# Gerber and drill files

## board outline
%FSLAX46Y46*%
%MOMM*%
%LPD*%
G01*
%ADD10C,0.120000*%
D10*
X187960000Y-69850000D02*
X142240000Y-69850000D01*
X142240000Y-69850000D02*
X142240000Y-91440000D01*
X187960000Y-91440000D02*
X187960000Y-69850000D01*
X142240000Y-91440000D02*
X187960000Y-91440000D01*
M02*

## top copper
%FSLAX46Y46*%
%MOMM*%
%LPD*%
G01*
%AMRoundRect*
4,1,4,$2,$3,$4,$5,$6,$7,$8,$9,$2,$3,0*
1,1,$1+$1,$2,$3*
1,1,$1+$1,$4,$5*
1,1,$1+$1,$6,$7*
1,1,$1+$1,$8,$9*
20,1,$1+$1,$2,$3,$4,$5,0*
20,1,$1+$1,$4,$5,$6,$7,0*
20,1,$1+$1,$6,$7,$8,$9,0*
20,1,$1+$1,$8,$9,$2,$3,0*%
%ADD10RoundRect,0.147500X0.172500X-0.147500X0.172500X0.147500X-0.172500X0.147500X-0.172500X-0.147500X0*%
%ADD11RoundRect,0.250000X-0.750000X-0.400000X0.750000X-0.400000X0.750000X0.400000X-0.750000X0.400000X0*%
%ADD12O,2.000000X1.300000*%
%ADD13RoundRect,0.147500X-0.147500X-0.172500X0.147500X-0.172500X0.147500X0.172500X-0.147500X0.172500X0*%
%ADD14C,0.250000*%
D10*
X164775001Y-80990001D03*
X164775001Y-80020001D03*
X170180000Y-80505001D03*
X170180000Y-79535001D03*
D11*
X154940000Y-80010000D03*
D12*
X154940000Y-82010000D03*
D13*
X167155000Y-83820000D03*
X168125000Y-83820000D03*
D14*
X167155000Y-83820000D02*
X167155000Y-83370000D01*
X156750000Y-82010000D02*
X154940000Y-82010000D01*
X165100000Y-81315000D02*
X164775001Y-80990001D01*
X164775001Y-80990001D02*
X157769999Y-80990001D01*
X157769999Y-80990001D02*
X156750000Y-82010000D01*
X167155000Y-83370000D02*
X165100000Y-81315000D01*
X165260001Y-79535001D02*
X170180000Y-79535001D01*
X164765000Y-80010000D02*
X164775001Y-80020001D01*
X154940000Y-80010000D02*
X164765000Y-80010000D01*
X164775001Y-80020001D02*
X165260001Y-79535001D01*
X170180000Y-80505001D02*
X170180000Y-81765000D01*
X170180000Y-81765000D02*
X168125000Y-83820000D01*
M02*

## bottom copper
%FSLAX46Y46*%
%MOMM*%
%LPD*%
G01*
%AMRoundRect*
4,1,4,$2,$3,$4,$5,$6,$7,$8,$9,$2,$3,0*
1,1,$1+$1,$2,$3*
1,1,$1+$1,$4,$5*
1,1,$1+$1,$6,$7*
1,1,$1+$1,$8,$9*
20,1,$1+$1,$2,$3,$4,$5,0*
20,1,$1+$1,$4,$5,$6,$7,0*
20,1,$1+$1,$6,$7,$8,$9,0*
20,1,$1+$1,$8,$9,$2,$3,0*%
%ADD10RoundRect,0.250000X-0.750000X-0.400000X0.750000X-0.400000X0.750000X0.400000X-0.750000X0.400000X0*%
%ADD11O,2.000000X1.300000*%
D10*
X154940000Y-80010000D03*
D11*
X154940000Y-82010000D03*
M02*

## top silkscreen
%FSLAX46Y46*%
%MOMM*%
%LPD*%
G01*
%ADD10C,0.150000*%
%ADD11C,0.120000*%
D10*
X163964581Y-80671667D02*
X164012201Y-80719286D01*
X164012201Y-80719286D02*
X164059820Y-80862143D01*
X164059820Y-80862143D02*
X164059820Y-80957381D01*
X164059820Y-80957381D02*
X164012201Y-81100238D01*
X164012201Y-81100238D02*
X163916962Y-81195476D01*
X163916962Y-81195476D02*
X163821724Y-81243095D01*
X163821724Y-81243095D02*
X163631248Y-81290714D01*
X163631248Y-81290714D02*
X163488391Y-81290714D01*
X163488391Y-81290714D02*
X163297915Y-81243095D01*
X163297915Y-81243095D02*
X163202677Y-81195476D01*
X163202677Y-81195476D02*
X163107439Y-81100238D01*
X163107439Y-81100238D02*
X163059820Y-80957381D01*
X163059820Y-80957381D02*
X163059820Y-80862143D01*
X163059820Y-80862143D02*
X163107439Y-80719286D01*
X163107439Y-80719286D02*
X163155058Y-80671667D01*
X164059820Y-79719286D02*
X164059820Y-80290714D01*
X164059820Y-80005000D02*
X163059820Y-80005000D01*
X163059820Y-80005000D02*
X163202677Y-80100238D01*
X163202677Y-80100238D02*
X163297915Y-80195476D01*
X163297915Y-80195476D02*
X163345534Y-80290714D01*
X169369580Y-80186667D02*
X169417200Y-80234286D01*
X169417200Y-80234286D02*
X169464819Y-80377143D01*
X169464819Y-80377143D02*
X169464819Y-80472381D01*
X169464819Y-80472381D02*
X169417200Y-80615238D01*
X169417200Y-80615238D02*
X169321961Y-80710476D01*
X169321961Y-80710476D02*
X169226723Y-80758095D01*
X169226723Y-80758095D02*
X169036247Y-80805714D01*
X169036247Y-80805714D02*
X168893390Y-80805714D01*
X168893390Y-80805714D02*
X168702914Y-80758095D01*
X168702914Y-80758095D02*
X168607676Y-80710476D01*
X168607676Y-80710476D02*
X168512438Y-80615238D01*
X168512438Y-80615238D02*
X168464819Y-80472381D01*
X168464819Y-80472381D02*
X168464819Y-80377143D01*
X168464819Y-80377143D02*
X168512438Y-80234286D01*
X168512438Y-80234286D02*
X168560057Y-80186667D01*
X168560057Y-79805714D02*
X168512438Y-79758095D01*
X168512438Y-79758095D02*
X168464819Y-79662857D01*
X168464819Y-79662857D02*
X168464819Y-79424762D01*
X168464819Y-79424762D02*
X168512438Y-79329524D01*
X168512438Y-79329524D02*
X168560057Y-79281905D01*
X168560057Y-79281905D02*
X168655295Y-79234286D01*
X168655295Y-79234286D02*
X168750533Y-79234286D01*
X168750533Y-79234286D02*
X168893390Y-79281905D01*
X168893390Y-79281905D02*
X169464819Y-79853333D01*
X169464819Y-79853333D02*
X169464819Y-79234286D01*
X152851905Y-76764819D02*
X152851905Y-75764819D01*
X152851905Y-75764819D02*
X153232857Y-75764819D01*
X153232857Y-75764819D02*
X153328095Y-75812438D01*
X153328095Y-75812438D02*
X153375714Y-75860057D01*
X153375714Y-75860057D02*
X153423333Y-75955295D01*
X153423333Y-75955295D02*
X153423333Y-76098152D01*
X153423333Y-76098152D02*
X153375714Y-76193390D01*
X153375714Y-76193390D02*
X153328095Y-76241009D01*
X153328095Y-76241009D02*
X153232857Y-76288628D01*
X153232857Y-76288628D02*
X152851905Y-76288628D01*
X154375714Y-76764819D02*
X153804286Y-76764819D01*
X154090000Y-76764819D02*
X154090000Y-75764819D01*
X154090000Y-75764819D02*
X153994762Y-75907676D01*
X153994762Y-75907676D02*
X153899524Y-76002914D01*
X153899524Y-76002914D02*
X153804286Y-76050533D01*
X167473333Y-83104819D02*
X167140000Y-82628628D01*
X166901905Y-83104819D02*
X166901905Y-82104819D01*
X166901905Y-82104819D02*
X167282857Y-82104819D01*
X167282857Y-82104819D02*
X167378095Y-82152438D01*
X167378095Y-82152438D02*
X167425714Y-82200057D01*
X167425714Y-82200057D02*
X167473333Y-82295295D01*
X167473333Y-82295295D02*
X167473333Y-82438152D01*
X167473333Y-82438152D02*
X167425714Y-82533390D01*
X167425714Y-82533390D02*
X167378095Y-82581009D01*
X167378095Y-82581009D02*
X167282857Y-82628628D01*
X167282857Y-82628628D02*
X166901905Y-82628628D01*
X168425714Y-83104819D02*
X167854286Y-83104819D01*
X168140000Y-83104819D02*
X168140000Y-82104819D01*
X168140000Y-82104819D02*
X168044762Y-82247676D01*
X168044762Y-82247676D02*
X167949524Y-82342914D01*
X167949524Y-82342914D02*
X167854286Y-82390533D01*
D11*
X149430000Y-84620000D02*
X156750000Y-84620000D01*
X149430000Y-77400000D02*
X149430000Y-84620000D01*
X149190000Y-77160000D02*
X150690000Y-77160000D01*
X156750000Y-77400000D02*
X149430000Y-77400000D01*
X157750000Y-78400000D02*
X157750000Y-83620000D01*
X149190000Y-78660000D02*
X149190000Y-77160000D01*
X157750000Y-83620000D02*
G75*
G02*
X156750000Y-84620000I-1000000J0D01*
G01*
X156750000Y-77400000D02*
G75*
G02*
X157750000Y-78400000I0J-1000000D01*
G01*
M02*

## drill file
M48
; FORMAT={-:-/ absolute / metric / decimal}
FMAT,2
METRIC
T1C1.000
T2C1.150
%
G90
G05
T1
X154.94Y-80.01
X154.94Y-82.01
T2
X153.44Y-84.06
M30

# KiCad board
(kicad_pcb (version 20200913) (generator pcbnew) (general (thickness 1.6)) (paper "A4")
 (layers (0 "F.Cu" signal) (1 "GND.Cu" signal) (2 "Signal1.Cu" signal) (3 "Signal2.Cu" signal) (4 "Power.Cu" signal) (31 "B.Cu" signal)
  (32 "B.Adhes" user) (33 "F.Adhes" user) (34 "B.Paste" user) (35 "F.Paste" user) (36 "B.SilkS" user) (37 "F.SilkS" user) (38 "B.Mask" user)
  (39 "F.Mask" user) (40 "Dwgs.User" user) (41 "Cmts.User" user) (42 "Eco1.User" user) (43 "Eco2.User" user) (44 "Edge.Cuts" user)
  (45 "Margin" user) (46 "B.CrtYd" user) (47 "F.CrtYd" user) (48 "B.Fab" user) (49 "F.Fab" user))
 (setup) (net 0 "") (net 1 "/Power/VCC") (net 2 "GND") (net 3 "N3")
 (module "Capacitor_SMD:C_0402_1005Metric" (layer "F.Cu") (at 164.775001 80.505001 90)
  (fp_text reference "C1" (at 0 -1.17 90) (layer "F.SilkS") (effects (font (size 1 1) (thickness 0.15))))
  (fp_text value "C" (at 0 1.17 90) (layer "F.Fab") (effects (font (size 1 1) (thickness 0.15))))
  (pad "1" smd roundrect (at -0.485 0 90) (size 0.59 0.64) (layers "F.Cu" "F.Paste" "F.Mask") (roundrect_rratio 0.25) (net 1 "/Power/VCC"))
  (pad "2" smd roundrect (at 0.485 0 90) (size 0.59 0.64) (layers "F.Cu" "F.Paste" "F.Mask") (roundrect_rratio 0.25) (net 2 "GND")))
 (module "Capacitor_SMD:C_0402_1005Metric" (layer "F.Cu") (at 170.18 80.020001 90)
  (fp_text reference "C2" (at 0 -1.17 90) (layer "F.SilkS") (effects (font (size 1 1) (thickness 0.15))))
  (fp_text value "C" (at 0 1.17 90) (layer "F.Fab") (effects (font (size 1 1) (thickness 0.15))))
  (pad "1" smd roundrect (at -0.485 0 90) (size 0.59 0.64) (layers "F.Cu" "F.Paste" "F.Mask") (roundrect_rratio 0.25) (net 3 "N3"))
  (pad "2" smd roundrect (at 0.485 0 90) (size 0.59 0.64) (layers "F.Cu" "F.Paste" "F.Mask") (roundrect_rratio 0.25) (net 2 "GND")))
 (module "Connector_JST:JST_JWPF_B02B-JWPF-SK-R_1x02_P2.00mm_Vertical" (layer "F.Cu") (at 154.94 80.01)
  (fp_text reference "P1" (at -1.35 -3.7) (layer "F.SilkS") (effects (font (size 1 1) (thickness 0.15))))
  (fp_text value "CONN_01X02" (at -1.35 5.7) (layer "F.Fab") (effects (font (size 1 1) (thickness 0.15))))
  (fp_line (start -5.51 4.61) (end 1.81 4.61) (layer "F.SilkS") (width 0.12))
  (fp_line (start -5.51 -2.61) (end -5.51 4.61) (layer "F.SilkS") (width 0.12))
  (fp_line (start -5.75 -2.85) (end -4.25 -2.85) (layer "F.SilkS") (width 0.12))
  (fp_line (start 1.81 -2.61) (end -5.51 -2.61) (layer "F.SilkS") (width 0.12))
  (fp_line (start 2.81 -1.61) (end 2.81 3.61) (layer "F.SilkS") (width 0.12))
  (fp_line (start -5.75 -1.35) (end -5.75 -2.85) (layer "F.SilkS") (width 0.12))
  (fp_arc (start 1.81 3.61) (end 2.81 3.61) (angle 90) (layer "F.SilkS") (width 0.12))
  (fp_arc (start 1.81 -1.61) (end 1.81 -2.61) (angle 90) (layer "F.SilkS") (width 0.12))
  (pad "" np_thru_hole circle (at -1.5 4.05) (size 1.15 1.15) (drill 1.15) (layers *.Cu *.Mask))
  (pad "1" thru_hole roundrect (at 0 0) (size 2 1.3) (drill 1) (layers *.Cu *.Mask) (roundrect_rratio 0.192308) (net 2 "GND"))
  (pad "2" thru_hole oval (at 0 2) (size 2 1.3) (drill 1) (layers *.Cu *.Mask) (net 1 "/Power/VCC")))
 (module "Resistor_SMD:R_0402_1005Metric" (layer "F.Cu") (at 167.64 83.82)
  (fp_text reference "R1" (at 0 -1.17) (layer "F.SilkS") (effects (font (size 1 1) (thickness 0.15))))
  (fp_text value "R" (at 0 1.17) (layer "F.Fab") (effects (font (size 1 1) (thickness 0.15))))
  (pad "1" smd roundrect (at -0.485 0) (size 0.59 0.64) (layers "F.Cu" "F.Paste" "F.Mask") (roundrect_rratio 0.25) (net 1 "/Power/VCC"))
  (pad "2" smd roundrect (at 0.485 0) (size 0.59 0.64) (layers "F.Cu" "F.Paste" "F.Mask") (roundrect_rratio 0.25) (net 3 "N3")))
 (gr_line (start 187.96 69.85) (end 142.24 69.85) (layer "Edge.Cuts") (width 0.12))
 (gr_line (start 142.24 69.85) (end 142.24 91.44) (layer "Edge.Cuts") (width 0.12))
 (gr_line (start 187.96 91.44) (end 187.96 69.85) (layer "Edge.Cuts") (width 0.12))
 (gr_line (start 142.24 91.44) (end 187.96 91.44) (layer "Edge.Cuts") (width 0.12))
 (segment (start 167.155 83.82) (end 167.155 83.37) (width 0.25) (layer "F.Cu") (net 1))
 (segment (start 156.75 82.01) (end 154.94 82.01) (width 0.25) (layer "F.Cu") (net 1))
 (segment (start 165.1 81.315) (end 164.775001 80.990001) (width 0.25) (layer "F.Cu") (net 1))
 (segment (start 164.775001 80.990001) (end 157.769999 80.990001) (width 0.25) (layer "F.Cu") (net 1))
 (segment (start 157.769999 80.990001) (end 156.75 82.01) (width 0.25) (layer "F.Cu") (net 1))
 (segment (start 167.155 83.37) (end 165.1 81.315) (width 0.25) (layer "F.Cu") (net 1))
 (segment (start 180 88) (end 160 88) (width 0.25) (layer "Signal1.Cu") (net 1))
 (segment (start 179.9848 73) (end 160 73) (width 0.25) (layer "Signal1.Cu") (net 1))
 (segment (start 180 73.0152) (end 179.9848 73) (width 0.25) (layer "Signal1.Cu") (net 1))
 (segment (start 160 88) (end 160 82.0874) (width 0.25) (layer "Signal1.Cu") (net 1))
 (segment (start 180 88) (end 180 73.0152) (width 0.25) (layer "Signal1.Cu") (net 1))
 (segment (start 160 82.0874) (end 160 73) (width 0.25) (layer "Signal1.Cu") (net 1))
 (segment (start 159.9226 82.01) (end 160 82.0874) (width 0.25) (layer "Signal1.Cu") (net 1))
 (segment (start 154.94 82.01) (end 159.9226 82.01) (width 0.25) (layer "Signal1.Cu") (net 1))
 (segment (start 161 82.0314) (end 161 87) (width 0.25) (layer "Power.Cu") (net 1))
 (segment (start 154.94 82.01) (end 160.9786 82.01) (width 0.25) (layer "Power.Cu") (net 1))
 (segment (start 179 86.9888) (end 179 74) (width 0.25) (layer "Power.Cu") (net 1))
 (segment (start 161 74) (end 179 74) (width 0.25) (layer "Power.Cu") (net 1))
 (segment (start 161 87) (end 178.9888 87) (width 0.25) (layer "Power.Cu") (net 1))
 (segment (start 178.9888 87) (end 179 86.9888) (width 0.25) (layer "Power.Cu") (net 1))
 (segment (start 160.9786 82.01) (end 161 82.0314) (width 0.25) (layer "Power.Cu") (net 1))
 (segment (start 161 74) (end 161 82.0314) (width 0.25) (layer "Power.Cu") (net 1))
 (segment (start 165.260001 79.535001) (end 170.18 79.535001) (width 0.25) (layer "F.Cu") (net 2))
 (segment (start 164.765 80.01) (end 164.775001 80.020001) (width 0.25) (layer "F.Cu") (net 2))
 (segment (start 154.94 80.01) (end 164.765 80.01) (width 0.25) (layer "F.Cu") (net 2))
 (segment (start 164.775001 80.020001) (end 165.260001 79.535001) (width 0.25) (layer "F.Cu") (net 2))
 (segment (start 180 73) (end 180 88) (width 0.25) (layer "GND.Cu") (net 2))
 (segment (start 160 73) (end 180 73) (width 0.25) (layer "GND.Cu") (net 2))
 (segment (start 180 88) (end 160.009 88) (width 0.25) (layer "GND.Cu") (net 2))
 (segment (start 160.009 88) (end 160 87.991) (width 0.25) (layer "GND.Cu") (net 2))
 (segment (start 154.9708 79.9792) (end 154.94 80.01) (width 0.25) (layer "GND.Cu") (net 2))
 (segment (start 160 79.9792) (end 154.9708 79.9792) (width 0.25) (layer "GND.Cu") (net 2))
 (segment (start 160 79.9792) (end 160 73) (width 0.25) (layer "GND.Cu") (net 2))
 (segment (start 160 87.991) (end 160 79.9792) (width 0.25) (layer "GND.Cu") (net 2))
 (segment (start 179 87) (end 179 74) (width 0.25) (layer "Signal2.Cu") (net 2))
 (segment (start 154.94 80.01) (end 160.9852 80.01) (width 0.25) (layer "Signal2.Cu") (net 2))
 (segment (start 160.995 74) (end 161 74.005) (width 0.25) (layer "Signal2.Cu") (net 2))
 (segment (start 161 87) (end 179 87) (width 0.25) (layer "Signal2.Cu") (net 2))
 (segment (start 160.9852 80.01) (end 161 80.0248) (width 0.25) (layer "Signal2.Cu") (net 2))
 (segment (start 179 74) (end 160.995 74) (width 0.25) (layer "Signal2.Cu") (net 2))
 (segment (start 161 80.0248) (end 161 87) (width 0.25) (layer "Signal2.Cu") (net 2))
 (segment (start 161 74.005) (end 161 80.0248) (width 0.25) (layer "Signal2.Cu") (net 2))
 (segment (start 170.18 80.505001) (end 170.18 81.765) (width 0.25) (layer "F.Cu") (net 3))
 (segment (start 170.18 81.765) (end 168.125 83.82) (width 0.25) (layer "F.Cu") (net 3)))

